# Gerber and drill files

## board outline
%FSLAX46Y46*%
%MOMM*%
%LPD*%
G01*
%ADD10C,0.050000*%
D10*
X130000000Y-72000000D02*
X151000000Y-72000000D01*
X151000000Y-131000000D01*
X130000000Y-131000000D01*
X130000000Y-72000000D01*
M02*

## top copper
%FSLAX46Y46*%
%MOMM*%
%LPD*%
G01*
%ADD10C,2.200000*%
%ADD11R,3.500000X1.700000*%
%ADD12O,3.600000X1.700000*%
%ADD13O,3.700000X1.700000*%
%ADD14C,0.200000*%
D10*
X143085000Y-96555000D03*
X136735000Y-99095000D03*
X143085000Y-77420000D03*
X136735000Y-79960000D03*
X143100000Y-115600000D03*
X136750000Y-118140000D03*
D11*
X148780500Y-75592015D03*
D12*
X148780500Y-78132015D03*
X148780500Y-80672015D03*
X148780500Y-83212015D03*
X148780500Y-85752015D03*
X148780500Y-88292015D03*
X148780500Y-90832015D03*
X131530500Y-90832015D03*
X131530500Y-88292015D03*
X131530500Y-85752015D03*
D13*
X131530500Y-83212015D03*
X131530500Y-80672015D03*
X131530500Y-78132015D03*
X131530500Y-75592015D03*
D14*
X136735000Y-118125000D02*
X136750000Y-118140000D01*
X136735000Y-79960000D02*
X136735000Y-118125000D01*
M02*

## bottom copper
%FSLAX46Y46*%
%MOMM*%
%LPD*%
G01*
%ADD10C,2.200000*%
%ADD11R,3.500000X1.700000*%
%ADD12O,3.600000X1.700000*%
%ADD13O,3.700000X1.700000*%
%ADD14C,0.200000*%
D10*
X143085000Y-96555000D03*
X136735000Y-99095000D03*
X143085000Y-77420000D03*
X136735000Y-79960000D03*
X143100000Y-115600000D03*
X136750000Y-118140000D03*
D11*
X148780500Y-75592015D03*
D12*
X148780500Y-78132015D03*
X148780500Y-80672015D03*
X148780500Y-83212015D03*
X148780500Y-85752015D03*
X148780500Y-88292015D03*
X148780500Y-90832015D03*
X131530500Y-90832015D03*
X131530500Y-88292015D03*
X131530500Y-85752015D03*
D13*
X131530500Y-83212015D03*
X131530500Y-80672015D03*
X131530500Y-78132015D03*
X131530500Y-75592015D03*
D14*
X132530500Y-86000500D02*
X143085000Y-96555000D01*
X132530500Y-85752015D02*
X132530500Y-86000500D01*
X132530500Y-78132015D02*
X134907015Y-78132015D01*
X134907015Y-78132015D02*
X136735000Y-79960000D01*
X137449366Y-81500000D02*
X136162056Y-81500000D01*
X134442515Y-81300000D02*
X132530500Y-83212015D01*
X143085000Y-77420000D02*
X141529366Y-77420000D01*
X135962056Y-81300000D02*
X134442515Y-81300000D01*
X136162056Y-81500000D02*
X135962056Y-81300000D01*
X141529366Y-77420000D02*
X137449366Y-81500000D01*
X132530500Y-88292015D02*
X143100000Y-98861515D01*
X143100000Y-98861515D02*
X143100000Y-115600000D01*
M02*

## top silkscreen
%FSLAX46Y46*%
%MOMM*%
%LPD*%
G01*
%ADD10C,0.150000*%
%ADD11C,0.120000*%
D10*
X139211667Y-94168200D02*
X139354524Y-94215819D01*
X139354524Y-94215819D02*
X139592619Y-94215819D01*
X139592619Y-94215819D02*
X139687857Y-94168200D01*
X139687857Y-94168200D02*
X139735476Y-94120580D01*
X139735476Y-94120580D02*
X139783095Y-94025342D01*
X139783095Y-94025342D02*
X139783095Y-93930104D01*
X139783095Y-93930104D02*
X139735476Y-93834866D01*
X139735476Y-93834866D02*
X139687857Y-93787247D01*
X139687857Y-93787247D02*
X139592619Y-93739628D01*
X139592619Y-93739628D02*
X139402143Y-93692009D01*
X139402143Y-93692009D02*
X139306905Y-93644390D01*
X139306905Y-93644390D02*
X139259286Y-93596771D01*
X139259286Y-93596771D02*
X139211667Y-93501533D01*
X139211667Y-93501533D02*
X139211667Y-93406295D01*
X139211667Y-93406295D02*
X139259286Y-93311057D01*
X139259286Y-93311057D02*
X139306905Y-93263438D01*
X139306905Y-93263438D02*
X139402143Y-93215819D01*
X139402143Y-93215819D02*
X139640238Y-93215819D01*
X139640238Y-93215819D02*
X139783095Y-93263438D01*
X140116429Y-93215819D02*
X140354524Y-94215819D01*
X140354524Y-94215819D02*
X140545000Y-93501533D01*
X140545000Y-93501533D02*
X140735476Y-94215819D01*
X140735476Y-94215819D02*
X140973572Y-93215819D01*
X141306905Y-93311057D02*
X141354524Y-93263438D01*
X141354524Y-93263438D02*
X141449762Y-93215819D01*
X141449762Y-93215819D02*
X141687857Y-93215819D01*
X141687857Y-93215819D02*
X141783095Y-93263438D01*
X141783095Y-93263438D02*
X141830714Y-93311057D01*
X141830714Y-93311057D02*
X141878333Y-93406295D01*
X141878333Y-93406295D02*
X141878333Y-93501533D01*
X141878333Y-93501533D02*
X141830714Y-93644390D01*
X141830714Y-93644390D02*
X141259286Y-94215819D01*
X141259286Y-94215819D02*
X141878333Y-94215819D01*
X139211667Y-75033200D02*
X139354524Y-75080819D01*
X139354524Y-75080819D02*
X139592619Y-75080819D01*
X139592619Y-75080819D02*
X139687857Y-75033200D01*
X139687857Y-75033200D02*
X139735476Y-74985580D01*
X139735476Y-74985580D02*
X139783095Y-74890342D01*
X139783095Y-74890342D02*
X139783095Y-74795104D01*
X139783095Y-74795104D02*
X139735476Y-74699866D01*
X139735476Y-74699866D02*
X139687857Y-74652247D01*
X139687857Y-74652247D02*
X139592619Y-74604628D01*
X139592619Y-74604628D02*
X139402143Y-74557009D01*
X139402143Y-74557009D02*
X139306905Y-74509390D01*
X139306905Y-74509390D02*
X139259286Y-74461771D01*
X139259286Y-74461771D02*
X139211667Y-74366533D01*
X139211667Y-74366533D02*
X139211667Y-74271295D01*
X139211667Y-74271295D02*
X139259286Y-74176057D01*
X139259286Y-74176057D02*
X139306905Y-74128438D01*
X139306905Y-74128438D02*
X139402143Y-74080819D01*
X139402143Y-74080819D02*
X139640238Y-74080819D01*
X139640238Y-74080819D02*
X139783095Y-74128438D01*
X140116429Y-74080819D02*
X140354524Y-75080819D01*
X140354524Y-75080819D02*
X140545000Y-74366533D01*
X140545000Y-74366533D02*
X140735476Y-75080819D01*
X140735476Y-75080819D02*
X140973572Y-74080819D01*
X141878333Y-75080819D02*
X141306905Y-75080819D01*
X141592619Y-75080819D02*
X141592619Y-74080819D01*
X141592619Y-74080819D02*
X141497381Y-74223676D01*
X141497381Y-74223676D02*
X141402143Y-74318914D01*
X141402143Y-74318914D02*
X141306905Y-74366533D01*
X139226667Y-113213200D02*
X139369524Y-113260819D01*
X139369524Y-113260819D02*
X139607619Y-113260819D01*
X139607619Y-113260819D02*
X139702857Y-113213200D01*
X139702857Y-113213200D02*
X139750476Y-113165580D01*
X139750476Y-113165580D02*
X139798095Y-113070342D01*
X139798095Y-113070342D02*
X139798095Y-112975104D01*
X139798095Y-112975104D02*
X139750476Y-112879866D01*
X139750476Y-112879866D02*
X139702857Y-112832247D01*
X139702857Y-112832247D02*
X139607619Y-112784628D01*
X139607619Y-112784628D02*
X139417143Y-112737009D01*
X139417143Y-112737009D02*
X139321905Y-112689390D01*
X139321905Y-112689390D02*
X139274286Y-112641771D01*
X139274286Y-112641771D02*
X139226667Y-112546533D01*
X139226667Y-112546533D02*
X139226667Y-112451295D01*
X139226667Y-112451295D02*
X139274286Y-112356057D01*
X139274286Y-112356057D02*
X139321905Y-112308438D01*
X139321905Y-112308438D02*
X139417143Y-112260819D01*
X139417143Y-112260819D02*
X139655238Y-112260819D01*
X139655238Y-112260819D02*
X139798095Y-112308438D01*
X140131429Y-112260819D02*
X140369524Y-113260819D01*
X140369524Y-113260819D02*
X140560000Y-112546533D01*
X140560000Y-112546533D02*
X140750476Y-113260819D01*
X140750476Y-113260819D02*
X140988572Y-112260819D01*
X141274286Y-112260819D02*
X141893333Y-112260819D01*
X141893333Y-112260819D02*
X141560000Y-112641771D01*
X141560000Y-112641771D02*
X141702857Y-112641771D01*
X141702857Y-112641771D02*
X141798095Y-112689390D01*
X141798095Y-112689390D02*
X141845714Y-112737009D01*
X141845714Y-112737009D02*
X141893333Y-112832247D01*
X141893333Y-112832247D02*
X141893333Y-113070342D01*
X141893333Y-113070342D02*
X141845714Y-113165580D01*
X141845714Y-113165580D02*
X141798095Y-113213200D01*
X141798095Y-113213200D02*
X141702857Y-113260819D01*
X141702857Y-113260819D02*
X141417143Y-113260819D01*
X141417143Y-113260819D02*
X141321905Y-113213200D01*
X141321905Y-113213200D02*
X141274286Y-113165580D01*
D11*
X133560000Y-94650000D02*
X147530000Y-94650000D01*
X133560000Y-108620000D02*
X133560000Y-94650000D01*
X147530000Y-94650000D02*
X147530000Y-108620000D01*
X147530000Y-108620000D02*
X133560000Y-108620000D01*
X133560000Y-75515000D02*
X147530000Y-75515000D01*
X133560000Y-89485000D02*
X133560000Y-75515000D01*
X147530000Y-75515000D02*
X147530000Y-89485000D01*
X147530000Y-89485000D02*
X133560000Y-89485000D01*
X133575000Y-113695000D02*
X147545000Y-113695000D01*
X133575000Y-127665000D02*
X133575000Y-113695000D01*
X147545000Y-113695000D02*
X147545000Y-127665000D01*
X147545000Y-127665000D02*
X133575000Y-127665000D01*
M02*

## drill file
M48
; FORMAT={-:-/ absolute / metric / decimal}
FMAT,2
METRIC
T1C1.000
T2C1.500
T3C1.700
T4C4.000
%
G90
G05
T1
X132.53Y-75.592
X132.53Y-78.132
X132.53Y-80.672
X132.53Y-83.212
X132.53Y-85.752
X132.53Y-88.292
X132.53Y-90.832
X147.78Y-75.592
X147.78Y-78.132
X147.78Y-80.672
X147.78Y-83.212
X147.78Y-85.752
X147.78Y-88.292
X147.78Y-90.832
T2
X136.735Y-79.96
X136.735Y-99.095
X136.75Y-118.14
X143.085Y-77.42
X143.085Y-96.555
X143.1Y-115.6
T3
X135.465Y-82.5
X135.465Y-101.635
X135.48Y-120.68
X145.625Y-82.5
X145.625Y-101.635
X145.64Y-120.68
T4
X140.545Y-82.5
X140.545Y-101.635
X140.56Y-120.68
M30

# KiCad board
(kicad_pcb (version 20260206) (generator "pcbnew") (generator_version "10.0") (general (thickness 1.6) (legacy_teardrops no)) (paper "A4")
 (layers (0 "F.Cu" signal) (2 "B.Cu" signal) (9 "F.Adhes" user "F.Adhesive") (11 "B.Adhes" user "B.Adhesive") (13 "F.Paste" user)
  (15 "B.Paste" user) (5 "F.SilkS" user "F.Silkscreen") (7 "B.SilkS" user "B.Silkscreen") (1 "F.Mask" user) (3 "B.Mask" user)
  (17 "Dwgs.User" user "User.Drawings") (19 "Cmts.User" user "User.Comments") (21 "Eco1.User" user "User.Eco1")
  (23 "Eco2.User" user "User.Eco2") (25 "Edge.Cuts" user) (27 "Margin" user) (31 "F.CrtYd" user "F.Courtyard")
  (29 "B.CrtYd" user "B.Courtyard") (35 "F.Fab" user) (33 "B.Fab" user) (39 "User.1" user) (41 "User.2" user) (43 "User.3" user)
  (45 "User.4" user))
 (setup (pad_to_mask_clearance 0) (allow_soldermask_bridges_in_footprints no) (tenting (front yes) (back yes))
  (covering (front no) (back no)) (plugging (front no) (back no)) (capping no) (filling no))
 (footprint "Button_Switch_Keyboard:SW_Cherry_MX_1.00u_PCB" (layer "F.Cu") (at 143.085 96.555)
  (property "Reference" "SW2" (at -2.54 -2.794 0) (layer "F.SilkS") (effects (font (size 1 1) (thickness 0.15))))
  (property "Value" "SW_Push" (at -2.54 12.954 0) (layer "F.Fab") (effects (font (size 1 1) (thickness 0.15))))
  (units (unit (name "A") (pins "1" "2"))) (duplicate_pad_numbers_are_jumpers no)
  (fp_line (start -9.525 -1.905) (end 4.445 -1.905) (stroke (width 0.12) (type solid)) (layer "F.SilkS"))
  (fp_line (start -9.525 12.065) (end -9.525 -1.905) (stroke (width 0.12) (type solid)) (layer "F.SilkS"))
  (fp_line (start 4.445 -1.905) (end 4.445 12.065) (stroke (width 0.12) (type solid)) (layer "F.SilkS"))
  (fp_line (start 4.445 12.065) (end -9.525 12.065) (stroke (width 0.12) (type solid)) (layer "F.SilkS"))
  (pad "" np_thru_hole circle (at -7.62 5.08) (size 1.7 1.7) (drill 1.7) (layers "*.Cu" "*.Mask"))
  (pad "" np_thru_hole circle (at -2.54 5.08) (size 4 4) (drill 4) (layers "*.Cu" "*.Mask"))
  (pad "" np_thru_hole circle (at 2.54 5.08) (size 1.7 1.7) (drill 1.7) (layers "*.Cu" "*.Mask"))
  (pad "1" thru_hole circle (at 0 0) (size 2.2 2.2) (drill 1.5) (layers "*.Cu" "*.Mask") (remove_unused_layers no)
   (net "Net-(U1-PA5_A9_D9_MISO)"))
  (pad "2" thru_hole circle (at -6.35 2.54) (size 2.2 2.2) (drill 1.5) (layers "*.Cu" "*.Mask") (remove_unused_layers no) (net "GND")))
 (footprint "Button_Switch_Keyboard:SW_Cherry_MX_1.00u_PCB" (layer "F.Cu") (at 143.085 77.42)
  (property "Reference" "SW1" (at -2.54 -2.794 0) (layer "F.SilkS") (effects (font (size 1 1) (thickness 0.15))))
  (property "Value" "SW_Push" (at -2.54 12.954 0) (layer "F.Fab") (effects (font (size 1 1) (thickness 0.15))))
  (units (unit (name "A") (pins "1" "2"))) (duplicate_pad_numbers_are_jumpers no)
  (fp_line (start -9.525 -1.905) (end 4.445 -1.905) (stroke (width 0.12) (type solid)) (layer "F.SilkS"))
  (fp_line (start -9.525 12.065) (end -9.525 -1.905) (stroke (width 0.12) (type solid)) (layer "F.SilkS"))
  (fp_line (start 4.445 -1.905) (end 4.445 12.065) (stroke (width 0.12) (type solid)) (layer "F.SilkS"))
  (fp_line (start 4.445 12.065) (end -9.525 12.065) (stroke (width 0.12) (type solid)) (layer "F.SilkS"))
  (pad "" np_thru_hole circle (at -7.62 5.08) (size 1.7 1.7) (drill 1.7) (layers "*.Cu" "*.Mask"))
  (pad "" np_thru_hole circle (at -2.54 5.08) (size 4 4) (drill 4) (layers "*.Cu" "*.Mask"))
  (pad "" np_thru_hole circle (at 2.54 5.08) (size 1.7 1.7) (drill 1.7) (layers "*.Cu" "*.Mask"))
  (pad "1" thru_hole circle (at 0 0) (size 2.2 2.2) (drill 1.5) (layers "*.Cu" "*.Mask") (remove_unused_layers no)
   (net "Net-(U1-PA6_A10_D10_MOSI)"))
  (pad "2" thru_hole circle (at -6.35 2.54) (size 2.2 2.2) (drill 1.5) (layers "*.Cu" "*.Mask") (remove_unused_layers no) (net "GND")))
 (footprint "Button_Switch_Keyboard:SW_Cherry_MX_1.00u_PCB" (layer "F.Cu") (at 143.1 115.6)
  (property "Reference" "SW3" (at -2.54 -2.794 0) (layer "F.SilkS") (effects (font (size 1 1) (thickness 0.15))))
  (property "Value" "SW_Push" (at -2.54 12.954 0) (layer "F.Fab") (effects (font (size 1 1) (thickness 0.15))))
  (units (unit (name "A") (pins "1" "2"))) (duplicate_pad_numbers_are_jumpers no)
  (fp_line (start -9.525 -1.905) (end 4.445 -1.905) (stroke (width 0.12) (type solid)) (layer "F.SilkS"))
  (fp_line (start -9.525 12.065) (end -9.525 -1.905) (stroke (width 0.12) (type solid)) (layer "F.SilkS"))
  (fp_line (start 4.445 -1.905) (end 4.445 12.065) (stroke (width 0.12) (type solid)) (layer "F.SilkS"))
  (fp_line (start 4.445 12.065) (end -9.525 12.065) (stroke (width 0.12) (type solid)) (layer "F.SilkS"))
  (pad "" np_thru_hole circle (at -7.62 5.08) (size 1.7 1.7) (drill 1.7) (layers "*.Cu" "*.Mask"))
  (pad "" np_thru_hole circle (at -2.54 5.08) (size 4 4) (drill 4) (layers "*.Cu" "*.Mask"))
  (pad "" np_thru_hole circle (at 2.54 5.08) (size 1.7 1.7) (drill 1.7) (layers "*.Cu" "*.Mask"))
  (pad "1" thru_hole circle (at 0 0) (size 2.2 2.2) (drill 1.5) (layers "*.Cu" "*.Mask") (remove_unused_layers no)
   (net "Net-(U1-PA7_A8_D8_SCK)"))
  (pad "2" thru_hole circle (at -6.35 2.54) (size 2.2 2.2) (drill 1.5) (layers "*.Cu" "*.Mask") (remove_unused_layers no) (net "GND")))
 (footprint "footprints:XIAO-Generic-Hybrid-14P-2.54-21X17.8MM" (layer "B.Cu") (at 140.1555 83.212015 180)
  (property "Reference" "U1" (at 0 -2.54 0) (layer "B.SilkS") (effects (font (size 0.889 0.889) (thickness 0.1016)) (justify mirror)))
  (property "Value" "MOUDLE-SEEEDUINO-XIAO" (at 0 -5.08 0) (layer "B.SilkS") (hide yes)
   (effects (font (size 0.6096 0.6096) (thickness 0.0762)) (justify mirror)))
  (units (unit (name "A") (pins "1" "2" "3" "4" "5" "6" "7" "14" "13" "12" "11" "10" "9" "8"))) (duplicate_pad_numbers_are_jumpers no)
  (pad "1" thru_hole rect (at -7.625 7.62 180) (size 3.5 1.7) (drill 1 (offset -1 0)) (layers "*.Cu" "*.Mask") (remove_unused_layers no)
   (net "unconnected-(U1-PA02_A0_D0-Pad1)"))
  (pad "2" thru_hole oval (at -7.625 5.08 180) (size 3.6 1.7) (drill 1 (offset -1 0)) (layers "*.Cu" "*.Mask") (remove_unused_layers no)
   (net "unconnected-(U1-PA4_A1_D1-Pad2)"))
  (pad "3" thru_hole oval (at -7.625 2.54 180) (size 3.6 1.7) (drill 1 (offset -1 0)) (layers "*.Cu" "*.Mask") (remove_unused_layers no)
   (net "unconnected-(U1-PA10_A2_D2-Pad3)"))
  (pad "4" thru_hole oval (at -7.625 0 180) (size 3.6 1.7) (drill 1 (offset -1 0)) (layers "*.Cu" "*.Mask") (remove_unused_layers no)
   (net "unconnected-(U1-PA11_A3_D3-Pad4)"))
  (pad "5" thru_hole oval (at -7.625 -2.54 180) (size 3.6 1.7) (drill 1 (offset -1 0)) (layers "*.Cu" "*.Mask") (remove_unused_layers no)
   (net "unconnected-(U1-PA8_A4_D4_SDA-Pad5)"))
  (pad "6" thru_hole oval (at -7.625 -5.08) (size 3.6 1.7) (drill 1 (offset 1 0)) (layers "*.Cu" "*.Mask") (remove_unused_layers no)
   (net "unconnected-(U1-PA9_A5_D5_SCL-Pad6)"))
  (pad "7" thru_hole oval (at -7.625 -7.62 180) (size 3.6 1.7) (drill 1 (offset -1 0)) (layers "*.Cu" "*.Mask") (remove_unused_layers no)
   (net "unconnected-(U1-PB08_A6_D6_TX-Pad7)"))
  (pad "8" thru_hole oval (at 7.625 -7.62 180) (size 3.6 1.7) (drill 1 (offset 1 0)) (layers "*.Cu" "*.Mask") (remove_unused_layers no)
   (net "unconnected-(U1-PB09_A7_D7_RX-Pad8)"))
  (pad "9" thru_hole oval (at 7.625 -5.08 180) (size 3.6 1.7) (drill 1 (offset 1 0)) (layers "*.Cu" "*.Mask") (remove_unused_layers no)
   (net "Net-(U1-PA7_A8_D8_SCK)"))
  (pad "10" thru_hole oval (at 7.625 -2.54 180) (size 3.6 1.7) (drill 1 (offset 1 0)) (layers "*.Cu" "*.Mask") (remove_unused_layers no)
   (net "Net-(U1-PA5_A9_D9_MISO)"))
  (pad "11" thru_hole oval (at 7.625 0 180) (size 3.7 1.7) (drill 1 (offset 1 0)) (layers "*.Cu" "*.Mask") (remove_unused_layers no)
   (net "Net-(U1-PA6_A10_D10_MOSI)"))
  (pad "12" thru_hole oval (at 7.625 2.54 180) (size 3.7 1.7) (drill 1 (offset 1 0)) (layers "*.Cu" "*.Mask") (remove_unused_layers no)
   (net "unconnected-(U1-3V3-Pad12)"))
  (pad "13" thru_hole oval (at 7.625 5.08 180) (size 3.7 1.7) (drill 1 (offset 1 0)) (layers "*.Cu" "*.Mask") (remove_unused_layers no)
   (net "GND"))
  (pad "14" thru_hole oval (at 7.625 7.62 180) (size 3.7 1.7) (drill 1 (offset 1 0)) (layers "*.Cu" "*.Mask") (remove_unused_layers no)
   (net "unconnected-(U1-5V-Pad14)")))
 (gr_rect (start 130 72) (end 151 131) (stroke (width 0.05) (type default)) (fill no) (layer "Edge.Cuts"))
 (segment (start 132.5305 86.0005) (end 143.085 96.555) (width 0.2) (layer "B.Cu") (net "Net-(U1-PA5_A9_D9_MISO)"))
 (segment (start 132.5305 85.752015) (end 132.5305 86.0005) (width 0.2) (layer "B.Cu") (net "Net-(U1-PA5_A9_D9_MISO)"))
 (segment (start 136.735 118.125) (end 136.75 118.14) (width 0.2) (layer "F.Cu") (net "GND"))
 (segment (start 136.735 79.96) (end 136.735 118.125) (width 0.2) (layer "F.Cu") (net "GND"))
 (segment (start 132.5305 78.132015) (end 134.907015 78.132015) (width 0.2) (layer "B.Cu") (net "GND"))
 (segment (start 134.907015 78.132015) (end 136.735 79.96) (width 0.2) (layer "B.Cu") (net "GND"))
 (segment (start 137.449366 81.5) (end 136.162056 81.5) (width 0.2) (layer "B.Cu") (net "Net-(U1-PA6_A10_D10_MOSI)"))
 (segment (start 134.442515 81.3) (end 132.5305 83.212015) (width 0.2) (layer "B.Cu") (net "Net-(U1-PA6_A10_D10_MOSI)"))
 (segment (start 143.085 77.42) (end 141.529366 77.42) (width 0.2) (layer "B.Cu") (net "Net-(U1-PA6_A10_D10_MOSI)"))
 (segment (start 135.962056 81.3) (end 134.442515 81.3) (width 0.2) (layer "B.Cu") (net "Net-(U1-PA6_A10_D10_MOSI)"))
 (segment (start 136.162056 81.5) (end 135.962056 81.3) (width 0.2) (layer "B.Cu") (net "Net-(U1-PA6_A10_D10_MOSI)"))
 (segment (start 141.529366 77.42) (end 137.449366 81.5) (width 0.2) (layer "B.Cu") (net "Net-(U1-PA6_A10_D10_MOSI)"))
 (segment (start 132.5305 88.292015) (end 143.1 98.861515) (width 0.2) (layer "B.Cu") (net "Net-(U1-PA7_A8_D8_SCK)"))
 (segment (start 143.1 98.861515) (end 143.1 115.6) (width 0.2) (layer "B.Cu") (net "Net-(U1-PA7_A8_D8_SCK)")))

